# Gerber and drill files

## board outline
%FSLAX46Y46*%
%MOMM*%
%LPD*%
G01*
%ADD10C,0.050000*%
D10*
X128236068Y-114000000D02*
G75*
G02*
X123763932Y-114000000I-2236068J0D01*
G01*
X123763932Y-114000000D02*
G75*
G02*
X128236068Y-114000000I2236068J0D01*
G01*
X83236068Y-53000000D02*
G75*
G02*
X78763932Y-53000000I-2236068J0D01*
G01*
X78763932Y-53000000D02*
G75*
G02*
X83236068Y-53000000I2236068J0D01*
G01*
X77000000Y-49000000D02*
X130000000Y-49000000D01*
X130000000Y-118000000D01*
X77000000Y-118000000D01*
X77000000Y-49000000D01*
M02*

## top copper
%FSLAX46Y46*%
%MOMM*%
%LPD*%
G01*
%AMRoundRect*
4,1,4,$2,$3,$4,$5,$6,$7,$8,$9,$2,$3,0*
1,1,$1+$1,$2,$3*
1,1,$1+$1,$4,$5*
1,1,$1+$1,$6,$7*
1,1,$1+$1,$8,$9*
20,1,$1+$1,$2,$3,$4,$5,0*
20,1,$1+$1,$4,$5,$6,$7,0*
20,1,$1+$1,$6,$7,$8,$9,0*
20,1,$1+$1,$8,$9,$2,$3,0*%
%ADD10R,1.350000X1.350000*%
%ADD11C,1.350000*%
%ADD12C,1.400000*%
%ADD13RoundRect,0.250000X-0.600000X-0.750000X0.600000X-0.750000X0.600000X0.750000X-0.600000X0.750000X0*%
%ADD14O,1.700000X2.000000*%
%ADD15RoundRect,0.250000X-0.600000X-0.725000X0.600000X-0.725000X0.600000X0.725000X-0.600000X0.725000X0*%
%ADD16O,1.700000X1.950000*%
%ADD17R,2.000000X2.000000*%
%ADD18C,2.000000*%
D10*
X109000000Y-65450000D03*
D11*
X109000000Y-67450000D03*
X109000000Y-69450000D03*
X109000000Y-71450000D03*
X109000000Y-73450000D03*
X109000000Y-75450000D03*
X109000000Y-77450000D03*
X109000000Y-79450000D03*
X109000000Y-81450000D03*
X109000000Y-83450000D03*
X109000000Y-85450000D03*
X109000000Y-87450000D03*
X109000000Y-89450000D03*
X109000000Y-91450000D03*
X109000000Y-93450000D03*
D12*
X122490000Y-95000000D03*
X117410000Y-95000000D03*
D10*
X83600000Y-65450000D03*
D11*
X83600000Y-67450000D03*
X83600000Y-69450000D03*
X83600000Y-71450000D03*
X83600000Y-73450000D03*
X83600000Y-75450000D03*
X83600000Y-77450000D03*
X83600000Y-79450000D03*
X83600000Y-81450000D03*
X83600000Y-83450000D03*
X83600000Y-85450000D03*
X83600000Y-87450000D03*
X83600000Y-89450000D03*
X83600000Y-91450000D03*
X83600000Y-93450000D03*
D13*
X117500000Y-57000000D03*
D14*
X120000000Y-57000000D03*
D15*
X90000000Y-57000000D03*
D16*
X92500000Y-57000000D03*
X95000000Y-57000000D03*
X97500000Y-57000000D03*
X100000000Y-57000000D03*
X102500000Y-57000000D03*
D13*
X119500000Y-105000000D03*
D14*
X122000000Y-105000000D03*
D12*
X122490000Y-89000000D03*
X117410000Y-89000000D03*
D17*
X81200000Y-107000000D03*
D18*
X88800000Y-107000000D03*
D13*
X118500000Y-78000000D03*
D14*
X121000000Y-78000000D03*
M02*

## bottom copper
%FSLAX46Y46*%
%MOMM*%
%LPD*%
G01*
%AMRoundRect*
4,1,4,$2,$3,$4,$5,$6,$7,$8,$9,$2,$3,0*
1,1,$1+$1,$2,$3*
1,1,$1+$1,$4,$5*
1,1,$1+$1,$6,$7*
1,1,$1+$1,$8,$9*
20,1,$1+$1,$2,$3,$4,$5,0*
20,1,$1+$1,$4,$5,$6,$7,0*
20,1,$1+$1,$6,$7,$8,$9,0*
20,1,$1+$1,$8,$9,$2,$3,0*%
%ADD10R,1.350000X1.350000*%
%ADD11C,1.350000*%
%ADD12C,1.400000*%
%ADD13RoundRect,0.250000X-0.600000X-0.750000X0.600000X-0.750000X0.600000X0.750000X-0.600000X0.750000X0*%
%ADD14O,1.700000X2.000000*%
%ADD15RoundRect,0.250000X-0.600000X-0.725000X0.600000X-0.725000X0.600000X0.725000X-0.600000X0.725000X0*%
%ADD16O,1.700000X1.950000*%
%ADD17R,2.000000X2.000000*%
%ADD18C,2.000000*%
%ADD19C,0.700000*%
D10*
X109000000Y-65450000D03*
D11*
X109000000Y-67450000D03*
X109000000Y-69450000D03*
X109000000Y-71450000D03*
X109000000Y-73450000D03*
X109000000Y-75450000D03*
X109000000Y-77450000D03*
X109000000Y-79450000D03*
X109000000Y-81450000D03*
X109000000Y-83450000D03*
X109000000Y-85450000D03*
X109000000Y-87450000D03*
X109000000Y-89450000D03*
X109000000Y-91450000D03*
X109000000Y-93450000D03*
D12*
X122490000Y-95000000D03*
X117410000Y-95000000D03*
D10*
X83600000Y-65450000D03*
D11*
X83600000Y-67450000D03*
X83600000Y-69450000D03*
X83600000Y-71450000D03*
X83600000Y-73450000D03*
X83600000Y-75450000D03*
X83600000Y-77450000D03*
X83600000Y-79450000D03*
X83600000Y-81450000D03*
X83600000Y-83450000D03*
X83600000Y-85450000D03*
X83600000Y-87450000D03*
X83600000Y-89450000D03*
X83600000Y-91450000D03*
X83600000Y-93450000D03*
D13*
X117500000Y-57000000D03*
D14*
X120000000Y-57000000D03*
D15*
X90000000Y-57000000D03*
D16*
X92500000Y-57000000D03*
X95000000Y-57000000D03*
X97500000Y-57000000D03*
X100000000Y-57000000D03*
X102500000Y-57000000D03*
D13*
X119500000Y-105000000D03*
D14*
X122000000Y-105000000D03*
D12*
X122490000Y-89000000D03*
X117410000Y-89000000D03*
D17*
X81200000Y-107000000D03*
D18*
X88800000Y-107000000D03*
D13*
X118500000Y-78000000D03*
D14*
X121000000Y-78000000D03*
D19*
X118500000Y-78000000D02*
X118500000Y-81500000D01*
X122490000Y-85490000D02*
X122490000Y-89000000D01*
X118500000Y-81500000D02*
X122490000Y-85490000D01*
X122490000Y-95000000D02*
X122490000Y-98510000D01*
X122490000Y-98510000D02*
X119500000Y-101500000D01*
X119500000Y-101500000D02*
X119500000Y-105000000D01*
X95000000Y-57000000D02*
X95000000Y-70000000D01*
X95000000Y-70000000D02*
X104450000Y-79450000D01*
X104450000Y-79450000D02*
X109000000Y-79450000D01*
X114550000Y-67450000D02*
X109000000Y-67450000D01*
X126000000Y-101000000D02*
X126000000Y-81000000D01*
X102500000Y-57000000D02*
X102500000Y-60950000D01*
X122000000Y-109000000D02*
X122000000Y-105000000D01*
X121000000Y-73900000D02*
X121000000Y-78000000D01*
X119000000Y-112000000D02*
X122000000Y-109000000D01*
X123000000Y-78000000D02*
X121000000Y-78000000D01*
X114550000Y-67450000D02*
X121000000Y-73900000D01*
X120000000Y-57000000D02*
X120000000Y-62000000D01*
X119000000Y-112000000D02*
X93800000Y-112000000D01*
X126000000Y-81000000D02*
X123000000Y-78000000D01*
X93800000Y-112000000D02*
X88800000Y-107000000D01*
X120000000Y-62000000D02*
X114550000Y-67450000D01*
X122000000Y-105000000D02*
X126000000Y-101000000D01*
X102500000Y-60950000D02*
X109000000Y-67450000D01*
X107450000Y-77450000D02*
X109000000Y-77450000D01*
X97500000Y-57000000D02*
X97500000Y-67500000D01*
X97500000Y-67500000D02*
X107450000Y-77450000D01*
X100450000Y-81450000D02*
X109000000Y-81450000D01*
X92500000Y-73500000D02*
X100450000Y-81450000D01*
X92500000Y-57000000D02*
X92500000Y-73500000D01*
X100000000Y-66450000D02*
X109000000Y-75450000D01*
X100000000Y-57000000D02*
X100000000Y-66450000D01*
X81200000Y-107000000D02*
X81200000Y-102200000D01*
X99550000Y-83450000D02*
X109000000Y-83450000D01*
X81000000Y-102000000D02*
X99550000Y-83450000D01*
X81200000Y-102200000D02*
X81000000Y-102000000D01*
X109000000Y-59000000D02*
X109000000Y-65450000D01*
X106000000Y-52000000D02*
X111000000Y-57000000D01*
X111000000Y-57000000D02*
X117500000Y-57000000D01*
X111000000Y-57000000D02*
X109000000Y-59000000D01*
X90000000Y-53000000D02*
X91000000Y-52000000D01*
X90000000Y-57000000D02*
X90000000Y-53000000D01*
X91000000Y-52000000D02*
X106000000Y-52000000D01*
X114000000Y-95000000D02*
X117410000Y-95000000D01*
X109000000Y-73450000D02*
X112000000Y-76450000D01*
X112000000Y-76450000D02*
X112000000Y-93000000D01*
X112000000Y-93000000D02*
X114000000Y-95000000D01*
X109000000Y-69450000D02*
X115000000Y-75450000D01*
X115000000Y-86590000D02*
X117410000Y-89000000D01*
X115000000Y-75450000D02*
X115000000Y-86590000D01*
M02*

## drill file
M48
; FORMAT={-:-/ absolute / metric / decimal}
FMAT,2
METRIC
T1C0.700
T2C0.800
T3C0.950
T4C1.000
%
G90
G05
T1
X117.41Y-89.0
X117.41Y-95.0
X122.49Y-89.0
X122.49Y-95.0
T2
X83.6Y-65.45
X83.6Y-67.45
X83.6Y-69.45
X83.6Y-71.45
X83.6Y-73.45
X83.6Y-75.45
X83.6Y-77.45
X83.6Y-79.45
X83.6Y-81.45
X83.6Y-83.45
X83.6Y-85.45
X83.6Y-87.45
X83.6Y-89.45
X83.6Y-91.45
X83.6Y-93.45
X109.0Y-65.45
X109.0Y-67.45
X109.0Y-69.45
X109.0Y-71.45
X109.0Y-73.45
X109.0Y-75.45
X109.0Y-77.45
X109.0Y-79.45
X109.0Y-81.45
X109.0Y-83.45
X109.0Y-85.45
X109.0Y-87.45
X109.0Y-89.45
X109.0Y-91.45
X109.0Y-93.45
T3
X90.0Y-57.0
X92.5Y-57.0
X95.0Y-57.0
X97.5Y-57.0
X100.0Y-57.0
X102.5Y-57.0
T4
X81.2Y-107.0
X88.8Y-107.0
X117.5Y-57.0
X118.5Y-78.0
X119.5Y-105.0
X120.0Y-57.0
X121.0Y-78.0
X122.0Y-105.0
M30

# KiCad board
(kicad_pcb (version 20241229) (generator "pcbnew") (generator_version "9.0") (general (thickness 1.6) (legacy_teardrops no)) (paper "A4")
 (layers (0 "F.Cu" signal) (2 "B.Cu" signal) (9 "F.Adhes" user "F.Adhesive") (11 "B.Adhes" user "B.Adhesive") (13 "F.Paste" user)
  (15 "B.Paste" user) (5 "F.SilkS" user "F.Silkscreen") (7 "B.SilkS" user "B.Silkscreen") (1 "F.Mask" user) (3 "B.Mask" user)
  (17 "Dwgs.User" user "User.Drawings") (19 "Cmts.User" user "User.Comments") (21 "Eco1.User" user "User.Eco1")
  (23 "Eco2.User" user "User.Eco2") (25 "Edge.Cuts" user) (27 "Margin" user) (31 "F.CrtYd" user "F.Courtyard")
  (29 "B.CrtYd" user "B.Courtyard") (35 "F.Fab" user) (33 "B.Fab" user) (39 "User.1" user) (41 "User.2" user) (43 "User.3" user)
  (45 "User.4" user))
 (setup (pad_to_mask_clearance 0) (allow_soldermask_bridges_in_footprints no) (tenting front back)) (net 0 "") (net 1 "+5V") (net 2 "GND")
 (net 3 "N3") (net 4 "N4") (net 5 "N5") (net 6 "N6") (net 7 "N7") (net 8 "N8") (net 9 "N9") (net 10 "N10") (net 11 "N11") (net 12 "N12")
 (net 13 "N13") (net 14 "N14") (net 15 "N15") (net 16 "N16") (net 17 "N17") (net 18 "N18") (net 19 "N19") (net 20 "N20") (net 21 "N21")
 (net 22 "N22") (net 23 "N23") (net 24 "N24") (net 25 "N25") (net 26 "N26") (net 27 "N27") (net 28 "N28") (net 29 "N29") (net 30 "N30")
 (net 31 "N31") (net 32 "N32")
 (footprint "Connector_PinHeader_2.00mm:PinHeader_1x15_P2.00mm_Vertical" (layer "F.Cu") (at 109 65.45)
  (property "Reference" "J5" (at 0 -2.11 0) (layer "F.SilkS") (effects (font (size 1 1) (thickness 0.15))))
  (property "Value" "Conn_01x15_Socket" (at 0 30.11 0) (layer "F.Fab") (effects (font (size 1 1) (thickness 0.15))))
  (pad "1" thru_hole rect (at 0 0) (size 1.35 1.35) (drill 0.8) (layers "*.Cu" "*.Mask") (remove_unused_layers no) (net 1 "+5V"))
  (pad "2" thru_hole circle (at 0 2) (size 1.35 1.35) (drill 0.8) (layers "*.Cu" "*.Mask") (remove_unused_layers no) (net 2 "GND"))
  (pad "3" thru_hole circle (at 0 4) (size 1.35 1.35) (drill 0.8) (layers "*.Cu" "*.Mask") (remove_unused_layers no) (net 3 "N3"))
  (pad "4" thru_hole circle (at 0 6) (size 1.35 1.35) (drill 0.8) (layers "*.Cu" "*.Mask") (remove_unused_layers no) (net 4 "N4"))
  (pad "5" thru_hole circle (at 0 8) (size 1.35 1.35) (drill 0.8) (layers "*.Cu" "*.Mask") (remove_unused_layers no) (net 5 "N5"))
  (pad "6" thru_hole circle (at 0 10) (size 1.35 1.35) (drill 0.8) (layers "*.Cu" "*.Mask") (remove_unused_layers no) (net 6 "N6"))
  (pad "7" thru_hole circle (at 0 12) (size 1.35 1.35) (drill 0.8) (layers "*.Cu" "*.Mask") (remove_unused_layers no) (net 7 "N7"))
  (pad "8" thru_hole circle (at 0 14) (size 1.35 1.35) (drill 0.8) (layers "*.Cu" "*.Mask") (remove_unused_layers no) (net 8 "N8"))
  (pad "9" thru_hole circle (at 0 16) (size 1.35 1.35) (drill 0.8) (layers "*.Cu" "*.Mask") (remove_unused_layers no) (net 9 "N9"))
  (pad "10" thru_hole circle (at 0 18) (size 1.35 1.35) (drill 0.8) (layers "*.Cu" "*.Mask") (remove_unused_layers no) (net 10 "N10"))
  (pad "11" thru_hole circle (at 0 20) (size 1.35 1.35) (drill 0.8) (layers "*.Cu" "*.Mask") (remove_unused_layers no) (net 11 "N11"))
  (pad "12" thru_hole circle (at 0 22) (size 1.35 1.35) (drill 0.8) (layers "*.Cu" "*.Mask") (remove_unused_layers no) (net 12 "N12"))
  (pad "13" thru_hole circle (at 0 24) (size 1.35 1.35) (drill 0.8) (layers "*.Cu" "*.Mask") (remove_unused_layers no) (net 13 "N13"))
  (pad "14" thru_hole circle (at 0 26) (size 1.35 1.35) (drill 0.8) (layers "*.Cu" "*.Mask") (remove_unused_layers no) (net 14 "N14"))
  (pad "15" thru_hole circle (at 0 28) (size 1.35 1.35) (drill 0.8) (layers "*.Cu" "*.Mask") (remove_unused_layers no) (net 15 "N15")))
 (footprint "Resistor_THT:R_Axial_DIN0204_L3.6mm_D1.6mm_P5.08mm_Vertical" (layer "F.Cu") (at 122.49 95 180)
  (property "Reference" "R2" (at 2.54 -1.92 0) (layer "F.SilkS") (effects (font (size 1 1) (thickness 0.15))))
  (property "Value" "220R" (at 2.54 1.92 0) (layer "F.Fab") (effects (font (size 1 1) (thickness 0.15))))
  (pad "1" thru_hole circle (at 0 0 180) (size 1.4 1.4) (drill 0.7) (layers "*.Cu" "*.Mask") (remove_unused_layers no) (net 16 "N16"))
  (pad "2" thru_hole circle (at 5.08 0 180) (size 1.4 1.4) (drill 0.7) (layers "*.Cu" "*.Mask") (remove_unused_layers no) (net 5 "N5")))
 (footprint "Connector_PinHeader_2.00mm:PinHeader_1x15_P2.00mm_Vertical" (layer "F.Cu") (at 83.6 65.45)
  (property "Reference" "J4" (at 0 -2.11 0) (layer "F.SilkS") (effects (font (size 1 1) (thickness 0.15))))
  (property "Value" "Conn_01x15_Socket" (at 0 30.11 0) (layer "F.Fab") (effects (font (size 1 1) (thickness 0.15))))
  (pad "1" thru_hole rect (at 0 0) (size 1.35 1.35) (drill 0.8) (layers "*.Cu" "*.Mask") (remove_unused_layers no) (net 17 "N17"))
  (pad "2" thru_hole circle (at 0 2) (size 1.35 1.35) (drill 0.8) (layers "*.Cu" "*.Mask") (remove_unused_layers no) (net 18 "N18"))
  (pad "3" thru_hole circle (at 0 4) (size 1.35 1.35) (drill 0.8) (layers "*.Cu" "*.Mask") (remove_unused_layers no) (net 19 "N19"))
  (pad "4" thru_hole circle (at 0 6) (size 1.35 1.35) (drill 0.8) (layers "*.Cu" "*.Mask") (remove_unused_layers no) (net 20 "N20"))
  (pad "5" thru_hole circle (at 0 8) (size 1.35 1.35) (drill 0.8) (layers "*.Cu" "*.Mask") (remove_unused_layers no) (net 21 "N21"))
  (pad "6" thru_hole circle (at 0 10) (size 1.35 1.35) (drill 0.8) (layers "*.Cu" "*.Mask") (remove_unused_layers no) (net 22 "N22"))
  (pad "7" thru_hole circle (at 0 12) (size 1.35 1.35) (drill 0.8) (layers "*.Cu" "*.Mask") (remove_unused_layers no) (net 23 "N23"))
  (pad "8" thru_hole circle (at 0 14) (size 1.35 1.35) (drill 0.8) (layers "*.Cu" "*.Mask") (remove_unused_layers no) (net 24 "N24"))
  (pad "9" thru_hole circle (at 0 16) (size 1.35 1.35) (drill 0.8) (layers "*.Cu" "*.Mask") (remove_unused_layers no) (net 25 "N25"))
  (pad "10" thru_hole circle (at 0 18) (size 1.35 1.35) (drill 0.8) (layers "*.Cu" "*.Mask") (remove_unused_layers no) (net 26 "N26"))
  (pad "11" thru_hole circle (at 0 20) (size 1.35 1.35) (drill 0.8) (layers "*.Cu" "*.Mask") (remove_unused_layers no) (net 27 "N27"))
  (pad "12" thru_hole circle (at 0 22) (size 1.35 1.35) (drill 0.8) (layers "*.Cu" "*.Mask") (remove_unused_layers no) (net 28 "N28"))
  (pad "13" thru_hole circle (at 0 24) (size 1.35 1.35) (drill 0.8) (layers "*.Cu" "*.Mask") (remove_unused_layers no) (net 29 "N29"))
  (pad "14" thru_hole circle (at 0 26) (size 1.35 1.35) (drill 0.8) (layers "*.Cu" "*.Mask") (remove_unused_layers no) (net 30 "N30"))
  (pad "15" thru_hole circle (at 0 28) (size 1.35 1.35) (drill 0.8) (layers "*.Cu" "*.Mask") (remove_unused_layers no) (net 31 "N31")))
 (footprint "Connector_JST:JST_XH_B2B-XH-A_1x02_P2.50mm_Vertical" (layer "F.Cu") (at 117.5 57)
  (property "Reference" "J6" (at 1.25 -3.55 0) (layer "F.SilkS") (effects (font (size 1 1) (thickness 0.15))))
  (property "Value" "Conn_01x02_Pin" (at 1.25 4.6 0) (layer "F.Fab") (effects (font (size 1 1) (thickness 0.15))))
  (pad "1" thru_hole roundrect (at 0 0) (size 1.7 2) (drill 1) (layers "*.Cu" "*.Mask") (remove_unused_layers no)
   (roundrect_rratio 0.147059) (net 1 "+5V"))
  (pad "2" thru_hole oval (at 2.5 0) (size 1.7 2) (drill 1) (layers "*.Cu" "*.Mask") (remove_unused_layers no) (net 2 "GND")))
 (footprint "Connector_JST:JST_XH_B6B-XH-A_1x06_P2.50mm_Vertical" (layer "F.Cu") (at 90 57)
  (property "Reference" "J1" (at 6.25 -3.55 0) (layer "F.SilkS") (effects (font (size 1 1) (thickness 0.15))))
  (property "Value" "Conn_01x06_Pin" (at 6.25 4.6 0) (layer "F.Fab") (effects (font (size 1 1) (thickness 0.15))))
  (pad "1" thru_hole roundrect (at 0 0) (size 1.7 1.95) (drill 0.95) (layers "*.Cu" "*.Mask") (remove_unused_layers no)
   (roundrect_rratio 0.147059) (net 1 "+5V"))
  (pad "2" thru_hole oval (at 2.5 0) (size 1.7 1.95) (drill 0.95) (layers "*.Cu" "*.Mask") (remove_unused_layers no) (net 9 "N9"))
  (pad "3" thru_hole oval (at 5 0) (size 1.7 1.95) (drill 0.95) (layers "*.Cu" "*.Mask") (remove_unused_layers no) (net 8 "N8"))
  (pad "4" thru_hole oval (at 7.5 0) (size 1.7 1.95) (drill 0.95) (layers "*.Cu" "*.Mask") (remove_unused_layers no) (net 7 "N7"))
  (pad "5" thru_hole oval (at 10 0) (size 1.7 1.95) (drill 0.95) (layers "*.Cu" "*.Mask") (remove_unused_layers no) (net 6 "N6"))
  (pad "6" thru_hole oval (at 12.5 0) (size 1.7 1.95) (drill 0.95) (layers "*.Cu" "*.Mask") (remove_unused_layers no) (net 2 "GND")))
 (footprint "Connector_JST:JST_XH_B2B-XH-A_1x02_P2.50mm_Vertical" (layer "F.Cu") (at 119.5 105)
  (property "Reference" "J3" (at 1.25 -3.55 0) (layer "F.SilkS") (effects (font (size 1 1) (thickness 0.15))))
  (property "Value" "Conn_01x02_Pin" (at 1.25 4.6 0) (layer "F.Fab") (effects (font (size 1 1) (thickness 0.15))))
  (pad "1" thru_hole roundrect (at 0 0) (size 1.7 2) (drill 1) (layers "*.Cu" "*.Mask") (remove_unused_layers no)
   (roundrect_rratio 0.147059) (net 16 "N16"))
  (pad "2" thru_hole oval (at 2.5 0) (size 1.7 2) (drill 1) (layers "*.Cu" "*.Mask") (remove_unused_layers no) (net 2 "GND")))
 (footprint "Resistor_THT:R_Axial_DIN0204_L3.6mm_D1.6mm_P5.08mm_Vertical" (layer "F.Cu") (at 122.49 89 180)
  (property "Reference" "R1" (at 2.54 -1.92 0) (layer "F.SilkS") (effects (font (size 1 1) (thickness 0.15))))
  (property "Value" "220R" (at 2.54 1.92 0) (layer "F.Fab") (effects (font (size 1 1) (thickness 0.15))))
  (pad "1" thru_hole circle (at 0 0 180) (size 1.4 1.4) (drill 0.7) (layers "*.Cu" "*.Mask") (remove_unused_layers no) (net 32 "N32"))
  (pad "2" thru_hole circle (at 5.08 0 180) (size 1.4 1.4) (drill 0.7) (layers "*.Cu" "*.Mask") (remove_unused_layers no) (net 3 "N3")))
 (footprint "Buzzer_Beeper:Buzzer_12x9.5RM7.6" (layer "F.Cu") (at 81.2 107)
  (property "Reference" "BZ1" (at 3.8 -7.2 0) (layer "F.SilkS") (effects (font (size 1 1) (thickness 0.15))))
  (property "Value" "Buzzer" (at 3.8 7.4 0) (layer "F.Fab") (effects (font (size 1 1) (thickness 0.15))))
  (pad "1" thru_hole rect (at 0 0) (size 2 2) (drill 1) (layers "*.Cu" "*.Mask") (remove_unused_layers no) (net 10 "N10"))
  (pad "2" thru_hole circle (at 7.6 0) (size 2 2) (drill 1) (layers "*.Cu" "*.Mask") (remove_unused_layers no) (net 2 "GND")))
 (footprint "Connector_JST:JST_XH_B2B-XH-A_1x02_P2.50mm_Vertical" (layer "F.Cu") (at 118.5 78)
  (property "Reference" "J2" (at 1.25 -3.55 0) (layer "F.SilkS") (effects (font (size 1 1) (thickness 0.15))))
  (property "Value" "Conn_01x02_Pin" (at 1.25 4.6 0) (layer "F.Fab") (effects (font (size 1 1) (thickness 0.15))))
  (pad "1" thru_hole roundrect (at 0 0) (size 1.7 2) (drill 1) (layers "*.Cu" "*.Mask") (remove_unused_layers no)
   (roundrect_rratio 0.147059) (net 32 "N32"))
  (pad "2" thru_hole oval (at 2.5 0) (size 1.7 2) (drill 1) (layers "*.Cu" "*.Mask") (remove_unused_layers no) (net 2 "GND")))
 (gr_circle (center 126 114) (end 127 116) (stroke (width 0.05) (type default)) (fill no) (layer "Edge.Cuts"))
 (gr_circle (center 81 53) (end 82 55) (stroke (width 0.05) (type default)) (fill no) (layer "Edge.Cuts"))
 (gr_rect (start 77 49) (end 130 118) (stroke (width 0.05) (type default)) (fill no) (layer "Edge.Cuts"))
 (segment (start 118.5 78) (end 118.5 81.5) (width 0.7) (layer "B.Cu") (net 32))
 (segment (start 122.49 85.49) (end 122.49 89) (width 0.7) (layer "B.Cu") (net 32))
 (segment (start 118.5 81.5) (end 122.49 85.49) (width 0.7) (layer "B.Cu") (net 32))
 (segment (start 122.49 95) (end 122.49 98.51) (width 0.7) (layer "B.Cu") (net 16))
 (segment (start 122.49 98.51) (end 119.5 101.5) (width 0.7) (layer "B.Cu") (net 16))
 (segment (start 119.5 101.5) (end 119.5 105) (width 0.7) (layer "B.Cu") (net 16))
 (segment (start 95 57) (end 95 70) (width 0.7) (layer "B.Cu") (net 8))
 (segment (start 95 70) (end 104.45 79.45) (width 0.7) (layer "B.Cu") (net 8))
 (segment (start 104.45 79.45) (end 109 79.45) (width 0.7) (layer "B.Cu") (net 8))
 (segment (start 114.55 67.45) (end 109 67.45) (width 0.7) (layer "B.Cu") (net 2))
 (segment (start 126 101) (end 126 81) (width 0.7) (layer "B.Cu") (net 2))
 (segment (start 102.5 57) (end 102.5 60.95) (width 0.7) (layer "B.Cu") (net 2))
 (segment (start 122 109) (end 122 105) (width 0.7) (layer "B.Cu") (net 2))
 (segment (start 121 73.9) (end 121 78) (width 0.7) (layer "B.Cu") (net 2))
 (segment (start 119 112) (end 122 109) (width 0.7) (layer "B.Cu") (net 2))
 (segment (start 123 78) (end 121 78) (width 0.7) (layer "B.Cu") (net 2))
 (segment (start 114.55 67.45) (end 121 73.9) (width 0.7) (layer "B.Cu") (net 2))
 (segment (start 120 57) (end 120 62) (width 0.7) (layer "B.Cu") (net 2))
 (segment (start 119 112) (end 93.8 112) (width 0.7) (layer "B.Cu") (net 2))
 (segment (start 126 81) (end 123 78) (width 0.7) (layer "B.Cu") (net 2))
 (segment (start 93.8 112) (end 88.8 107) (width 0.7) (layer "B.Cu") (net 2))
 (segment (start 120 62) (end 114.55 67.45) (width 0.7) (layer "B.Cu") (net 2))
 (segment (start 122 105) (end 126 101) (width 0.7) (layer "B.Cu") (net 2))
 (segment (start 102.5 60.95) (end 109 67.45) (width 0.7) (layer "B.Cu") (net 2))
 (segment (start 107.45 77.45) (end 109 77.45) (width 0.7) (layer "B.Cu") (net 7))
 (segment (start 97.5 57) (end 97.5 67.5) (width 0.7) (layer "B.Cu") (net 7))
 (segment (start 97.5 67.5) (end 107.45 77.45) (width 0.7) (layer "B.Cu") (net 7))
 (segment (start 100.45 81.45) (end 109 81.45) (width 0.7) (layer "B.Cu") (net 9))
 (segment (start 92.5 73.5) (end 100.45 81.45) (width 0.7) (layer "B.Cu") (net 9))
 (segment (start 92.5 57) (end 92.5 73.5) (width 0.7) (layer "B.Cu") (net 9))
 (segment (start 100 66.45) (end 109 75.45) (width 0.7) (layer "B.Cu") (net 6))
 (segment (start 100 57) (end 100 66.45) (width 0.7) (layer "B.Cu") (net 6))
 (segment (start 81.2 107) (end 81.2 102.2) (width 0.7) (layer "B.Cu") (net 10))
 (segment (start 99.55 83.45) (end 109 83.45) (width 0.7) (layer "B.Cu") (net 10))
 (segment (start 81 102) (end 99.55 83.45) (width 0.7) (layer "B.Cu") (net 10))
 (segment (start 81.2 102.2) (end 81 102) (width 0.7) (layer "B.Cu") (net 10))
 (segment (start 109 59) (end 109 65.45) (width 0.7) (layer "B.Cu") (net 1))
 (segment (start 106 52) (end 111 57) (width 0.7) (layer "B.Cu") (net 1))
 (segment (start 111 57) (end 117.5 57) (width 0.7) (layer "B.Cu") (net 1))
 (segment (start 111 57) (end 109 59) (width 0.7) (layer "B.Cu") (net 1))
 (segment (start 90 53) (end 91 52) (width 0.7) (layer "B.Cu") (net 1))
 (segment (start 90 57) (end 90 53) (width 0.7) (layer "B.Cu") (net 1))
 (segment (start 91 52) (end 106 52) (width 0.7) (layer "B.Cu") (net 1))
 (segment (start 114 95) (end 117.41 95) (width 0.7) (layer "B.Cu") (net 5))
 (segment (start 109 73.45) (end 112 76.45) (width 0.7) (layer "B.Cu") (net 5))
 (segment (start 112 76.45) (end 112 93) (width 0.7) (layer "B.Cu") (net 5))
 (segment (start 112 93) (end 114 95) (width 0.7) (layer "B.Cu") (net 5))
 (segment (start 109 69.45) (end 115 75.45) (width 0.7) (layer "B.Cu") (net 3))
 (segment (start 115 86.59) (end 117.41 89) (width 0.7) (layer "B.Cu") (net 3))
 (segment (start 115 75.45) (end 115 86.59) (width 0.7) (layer "B.Cu") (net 3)))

